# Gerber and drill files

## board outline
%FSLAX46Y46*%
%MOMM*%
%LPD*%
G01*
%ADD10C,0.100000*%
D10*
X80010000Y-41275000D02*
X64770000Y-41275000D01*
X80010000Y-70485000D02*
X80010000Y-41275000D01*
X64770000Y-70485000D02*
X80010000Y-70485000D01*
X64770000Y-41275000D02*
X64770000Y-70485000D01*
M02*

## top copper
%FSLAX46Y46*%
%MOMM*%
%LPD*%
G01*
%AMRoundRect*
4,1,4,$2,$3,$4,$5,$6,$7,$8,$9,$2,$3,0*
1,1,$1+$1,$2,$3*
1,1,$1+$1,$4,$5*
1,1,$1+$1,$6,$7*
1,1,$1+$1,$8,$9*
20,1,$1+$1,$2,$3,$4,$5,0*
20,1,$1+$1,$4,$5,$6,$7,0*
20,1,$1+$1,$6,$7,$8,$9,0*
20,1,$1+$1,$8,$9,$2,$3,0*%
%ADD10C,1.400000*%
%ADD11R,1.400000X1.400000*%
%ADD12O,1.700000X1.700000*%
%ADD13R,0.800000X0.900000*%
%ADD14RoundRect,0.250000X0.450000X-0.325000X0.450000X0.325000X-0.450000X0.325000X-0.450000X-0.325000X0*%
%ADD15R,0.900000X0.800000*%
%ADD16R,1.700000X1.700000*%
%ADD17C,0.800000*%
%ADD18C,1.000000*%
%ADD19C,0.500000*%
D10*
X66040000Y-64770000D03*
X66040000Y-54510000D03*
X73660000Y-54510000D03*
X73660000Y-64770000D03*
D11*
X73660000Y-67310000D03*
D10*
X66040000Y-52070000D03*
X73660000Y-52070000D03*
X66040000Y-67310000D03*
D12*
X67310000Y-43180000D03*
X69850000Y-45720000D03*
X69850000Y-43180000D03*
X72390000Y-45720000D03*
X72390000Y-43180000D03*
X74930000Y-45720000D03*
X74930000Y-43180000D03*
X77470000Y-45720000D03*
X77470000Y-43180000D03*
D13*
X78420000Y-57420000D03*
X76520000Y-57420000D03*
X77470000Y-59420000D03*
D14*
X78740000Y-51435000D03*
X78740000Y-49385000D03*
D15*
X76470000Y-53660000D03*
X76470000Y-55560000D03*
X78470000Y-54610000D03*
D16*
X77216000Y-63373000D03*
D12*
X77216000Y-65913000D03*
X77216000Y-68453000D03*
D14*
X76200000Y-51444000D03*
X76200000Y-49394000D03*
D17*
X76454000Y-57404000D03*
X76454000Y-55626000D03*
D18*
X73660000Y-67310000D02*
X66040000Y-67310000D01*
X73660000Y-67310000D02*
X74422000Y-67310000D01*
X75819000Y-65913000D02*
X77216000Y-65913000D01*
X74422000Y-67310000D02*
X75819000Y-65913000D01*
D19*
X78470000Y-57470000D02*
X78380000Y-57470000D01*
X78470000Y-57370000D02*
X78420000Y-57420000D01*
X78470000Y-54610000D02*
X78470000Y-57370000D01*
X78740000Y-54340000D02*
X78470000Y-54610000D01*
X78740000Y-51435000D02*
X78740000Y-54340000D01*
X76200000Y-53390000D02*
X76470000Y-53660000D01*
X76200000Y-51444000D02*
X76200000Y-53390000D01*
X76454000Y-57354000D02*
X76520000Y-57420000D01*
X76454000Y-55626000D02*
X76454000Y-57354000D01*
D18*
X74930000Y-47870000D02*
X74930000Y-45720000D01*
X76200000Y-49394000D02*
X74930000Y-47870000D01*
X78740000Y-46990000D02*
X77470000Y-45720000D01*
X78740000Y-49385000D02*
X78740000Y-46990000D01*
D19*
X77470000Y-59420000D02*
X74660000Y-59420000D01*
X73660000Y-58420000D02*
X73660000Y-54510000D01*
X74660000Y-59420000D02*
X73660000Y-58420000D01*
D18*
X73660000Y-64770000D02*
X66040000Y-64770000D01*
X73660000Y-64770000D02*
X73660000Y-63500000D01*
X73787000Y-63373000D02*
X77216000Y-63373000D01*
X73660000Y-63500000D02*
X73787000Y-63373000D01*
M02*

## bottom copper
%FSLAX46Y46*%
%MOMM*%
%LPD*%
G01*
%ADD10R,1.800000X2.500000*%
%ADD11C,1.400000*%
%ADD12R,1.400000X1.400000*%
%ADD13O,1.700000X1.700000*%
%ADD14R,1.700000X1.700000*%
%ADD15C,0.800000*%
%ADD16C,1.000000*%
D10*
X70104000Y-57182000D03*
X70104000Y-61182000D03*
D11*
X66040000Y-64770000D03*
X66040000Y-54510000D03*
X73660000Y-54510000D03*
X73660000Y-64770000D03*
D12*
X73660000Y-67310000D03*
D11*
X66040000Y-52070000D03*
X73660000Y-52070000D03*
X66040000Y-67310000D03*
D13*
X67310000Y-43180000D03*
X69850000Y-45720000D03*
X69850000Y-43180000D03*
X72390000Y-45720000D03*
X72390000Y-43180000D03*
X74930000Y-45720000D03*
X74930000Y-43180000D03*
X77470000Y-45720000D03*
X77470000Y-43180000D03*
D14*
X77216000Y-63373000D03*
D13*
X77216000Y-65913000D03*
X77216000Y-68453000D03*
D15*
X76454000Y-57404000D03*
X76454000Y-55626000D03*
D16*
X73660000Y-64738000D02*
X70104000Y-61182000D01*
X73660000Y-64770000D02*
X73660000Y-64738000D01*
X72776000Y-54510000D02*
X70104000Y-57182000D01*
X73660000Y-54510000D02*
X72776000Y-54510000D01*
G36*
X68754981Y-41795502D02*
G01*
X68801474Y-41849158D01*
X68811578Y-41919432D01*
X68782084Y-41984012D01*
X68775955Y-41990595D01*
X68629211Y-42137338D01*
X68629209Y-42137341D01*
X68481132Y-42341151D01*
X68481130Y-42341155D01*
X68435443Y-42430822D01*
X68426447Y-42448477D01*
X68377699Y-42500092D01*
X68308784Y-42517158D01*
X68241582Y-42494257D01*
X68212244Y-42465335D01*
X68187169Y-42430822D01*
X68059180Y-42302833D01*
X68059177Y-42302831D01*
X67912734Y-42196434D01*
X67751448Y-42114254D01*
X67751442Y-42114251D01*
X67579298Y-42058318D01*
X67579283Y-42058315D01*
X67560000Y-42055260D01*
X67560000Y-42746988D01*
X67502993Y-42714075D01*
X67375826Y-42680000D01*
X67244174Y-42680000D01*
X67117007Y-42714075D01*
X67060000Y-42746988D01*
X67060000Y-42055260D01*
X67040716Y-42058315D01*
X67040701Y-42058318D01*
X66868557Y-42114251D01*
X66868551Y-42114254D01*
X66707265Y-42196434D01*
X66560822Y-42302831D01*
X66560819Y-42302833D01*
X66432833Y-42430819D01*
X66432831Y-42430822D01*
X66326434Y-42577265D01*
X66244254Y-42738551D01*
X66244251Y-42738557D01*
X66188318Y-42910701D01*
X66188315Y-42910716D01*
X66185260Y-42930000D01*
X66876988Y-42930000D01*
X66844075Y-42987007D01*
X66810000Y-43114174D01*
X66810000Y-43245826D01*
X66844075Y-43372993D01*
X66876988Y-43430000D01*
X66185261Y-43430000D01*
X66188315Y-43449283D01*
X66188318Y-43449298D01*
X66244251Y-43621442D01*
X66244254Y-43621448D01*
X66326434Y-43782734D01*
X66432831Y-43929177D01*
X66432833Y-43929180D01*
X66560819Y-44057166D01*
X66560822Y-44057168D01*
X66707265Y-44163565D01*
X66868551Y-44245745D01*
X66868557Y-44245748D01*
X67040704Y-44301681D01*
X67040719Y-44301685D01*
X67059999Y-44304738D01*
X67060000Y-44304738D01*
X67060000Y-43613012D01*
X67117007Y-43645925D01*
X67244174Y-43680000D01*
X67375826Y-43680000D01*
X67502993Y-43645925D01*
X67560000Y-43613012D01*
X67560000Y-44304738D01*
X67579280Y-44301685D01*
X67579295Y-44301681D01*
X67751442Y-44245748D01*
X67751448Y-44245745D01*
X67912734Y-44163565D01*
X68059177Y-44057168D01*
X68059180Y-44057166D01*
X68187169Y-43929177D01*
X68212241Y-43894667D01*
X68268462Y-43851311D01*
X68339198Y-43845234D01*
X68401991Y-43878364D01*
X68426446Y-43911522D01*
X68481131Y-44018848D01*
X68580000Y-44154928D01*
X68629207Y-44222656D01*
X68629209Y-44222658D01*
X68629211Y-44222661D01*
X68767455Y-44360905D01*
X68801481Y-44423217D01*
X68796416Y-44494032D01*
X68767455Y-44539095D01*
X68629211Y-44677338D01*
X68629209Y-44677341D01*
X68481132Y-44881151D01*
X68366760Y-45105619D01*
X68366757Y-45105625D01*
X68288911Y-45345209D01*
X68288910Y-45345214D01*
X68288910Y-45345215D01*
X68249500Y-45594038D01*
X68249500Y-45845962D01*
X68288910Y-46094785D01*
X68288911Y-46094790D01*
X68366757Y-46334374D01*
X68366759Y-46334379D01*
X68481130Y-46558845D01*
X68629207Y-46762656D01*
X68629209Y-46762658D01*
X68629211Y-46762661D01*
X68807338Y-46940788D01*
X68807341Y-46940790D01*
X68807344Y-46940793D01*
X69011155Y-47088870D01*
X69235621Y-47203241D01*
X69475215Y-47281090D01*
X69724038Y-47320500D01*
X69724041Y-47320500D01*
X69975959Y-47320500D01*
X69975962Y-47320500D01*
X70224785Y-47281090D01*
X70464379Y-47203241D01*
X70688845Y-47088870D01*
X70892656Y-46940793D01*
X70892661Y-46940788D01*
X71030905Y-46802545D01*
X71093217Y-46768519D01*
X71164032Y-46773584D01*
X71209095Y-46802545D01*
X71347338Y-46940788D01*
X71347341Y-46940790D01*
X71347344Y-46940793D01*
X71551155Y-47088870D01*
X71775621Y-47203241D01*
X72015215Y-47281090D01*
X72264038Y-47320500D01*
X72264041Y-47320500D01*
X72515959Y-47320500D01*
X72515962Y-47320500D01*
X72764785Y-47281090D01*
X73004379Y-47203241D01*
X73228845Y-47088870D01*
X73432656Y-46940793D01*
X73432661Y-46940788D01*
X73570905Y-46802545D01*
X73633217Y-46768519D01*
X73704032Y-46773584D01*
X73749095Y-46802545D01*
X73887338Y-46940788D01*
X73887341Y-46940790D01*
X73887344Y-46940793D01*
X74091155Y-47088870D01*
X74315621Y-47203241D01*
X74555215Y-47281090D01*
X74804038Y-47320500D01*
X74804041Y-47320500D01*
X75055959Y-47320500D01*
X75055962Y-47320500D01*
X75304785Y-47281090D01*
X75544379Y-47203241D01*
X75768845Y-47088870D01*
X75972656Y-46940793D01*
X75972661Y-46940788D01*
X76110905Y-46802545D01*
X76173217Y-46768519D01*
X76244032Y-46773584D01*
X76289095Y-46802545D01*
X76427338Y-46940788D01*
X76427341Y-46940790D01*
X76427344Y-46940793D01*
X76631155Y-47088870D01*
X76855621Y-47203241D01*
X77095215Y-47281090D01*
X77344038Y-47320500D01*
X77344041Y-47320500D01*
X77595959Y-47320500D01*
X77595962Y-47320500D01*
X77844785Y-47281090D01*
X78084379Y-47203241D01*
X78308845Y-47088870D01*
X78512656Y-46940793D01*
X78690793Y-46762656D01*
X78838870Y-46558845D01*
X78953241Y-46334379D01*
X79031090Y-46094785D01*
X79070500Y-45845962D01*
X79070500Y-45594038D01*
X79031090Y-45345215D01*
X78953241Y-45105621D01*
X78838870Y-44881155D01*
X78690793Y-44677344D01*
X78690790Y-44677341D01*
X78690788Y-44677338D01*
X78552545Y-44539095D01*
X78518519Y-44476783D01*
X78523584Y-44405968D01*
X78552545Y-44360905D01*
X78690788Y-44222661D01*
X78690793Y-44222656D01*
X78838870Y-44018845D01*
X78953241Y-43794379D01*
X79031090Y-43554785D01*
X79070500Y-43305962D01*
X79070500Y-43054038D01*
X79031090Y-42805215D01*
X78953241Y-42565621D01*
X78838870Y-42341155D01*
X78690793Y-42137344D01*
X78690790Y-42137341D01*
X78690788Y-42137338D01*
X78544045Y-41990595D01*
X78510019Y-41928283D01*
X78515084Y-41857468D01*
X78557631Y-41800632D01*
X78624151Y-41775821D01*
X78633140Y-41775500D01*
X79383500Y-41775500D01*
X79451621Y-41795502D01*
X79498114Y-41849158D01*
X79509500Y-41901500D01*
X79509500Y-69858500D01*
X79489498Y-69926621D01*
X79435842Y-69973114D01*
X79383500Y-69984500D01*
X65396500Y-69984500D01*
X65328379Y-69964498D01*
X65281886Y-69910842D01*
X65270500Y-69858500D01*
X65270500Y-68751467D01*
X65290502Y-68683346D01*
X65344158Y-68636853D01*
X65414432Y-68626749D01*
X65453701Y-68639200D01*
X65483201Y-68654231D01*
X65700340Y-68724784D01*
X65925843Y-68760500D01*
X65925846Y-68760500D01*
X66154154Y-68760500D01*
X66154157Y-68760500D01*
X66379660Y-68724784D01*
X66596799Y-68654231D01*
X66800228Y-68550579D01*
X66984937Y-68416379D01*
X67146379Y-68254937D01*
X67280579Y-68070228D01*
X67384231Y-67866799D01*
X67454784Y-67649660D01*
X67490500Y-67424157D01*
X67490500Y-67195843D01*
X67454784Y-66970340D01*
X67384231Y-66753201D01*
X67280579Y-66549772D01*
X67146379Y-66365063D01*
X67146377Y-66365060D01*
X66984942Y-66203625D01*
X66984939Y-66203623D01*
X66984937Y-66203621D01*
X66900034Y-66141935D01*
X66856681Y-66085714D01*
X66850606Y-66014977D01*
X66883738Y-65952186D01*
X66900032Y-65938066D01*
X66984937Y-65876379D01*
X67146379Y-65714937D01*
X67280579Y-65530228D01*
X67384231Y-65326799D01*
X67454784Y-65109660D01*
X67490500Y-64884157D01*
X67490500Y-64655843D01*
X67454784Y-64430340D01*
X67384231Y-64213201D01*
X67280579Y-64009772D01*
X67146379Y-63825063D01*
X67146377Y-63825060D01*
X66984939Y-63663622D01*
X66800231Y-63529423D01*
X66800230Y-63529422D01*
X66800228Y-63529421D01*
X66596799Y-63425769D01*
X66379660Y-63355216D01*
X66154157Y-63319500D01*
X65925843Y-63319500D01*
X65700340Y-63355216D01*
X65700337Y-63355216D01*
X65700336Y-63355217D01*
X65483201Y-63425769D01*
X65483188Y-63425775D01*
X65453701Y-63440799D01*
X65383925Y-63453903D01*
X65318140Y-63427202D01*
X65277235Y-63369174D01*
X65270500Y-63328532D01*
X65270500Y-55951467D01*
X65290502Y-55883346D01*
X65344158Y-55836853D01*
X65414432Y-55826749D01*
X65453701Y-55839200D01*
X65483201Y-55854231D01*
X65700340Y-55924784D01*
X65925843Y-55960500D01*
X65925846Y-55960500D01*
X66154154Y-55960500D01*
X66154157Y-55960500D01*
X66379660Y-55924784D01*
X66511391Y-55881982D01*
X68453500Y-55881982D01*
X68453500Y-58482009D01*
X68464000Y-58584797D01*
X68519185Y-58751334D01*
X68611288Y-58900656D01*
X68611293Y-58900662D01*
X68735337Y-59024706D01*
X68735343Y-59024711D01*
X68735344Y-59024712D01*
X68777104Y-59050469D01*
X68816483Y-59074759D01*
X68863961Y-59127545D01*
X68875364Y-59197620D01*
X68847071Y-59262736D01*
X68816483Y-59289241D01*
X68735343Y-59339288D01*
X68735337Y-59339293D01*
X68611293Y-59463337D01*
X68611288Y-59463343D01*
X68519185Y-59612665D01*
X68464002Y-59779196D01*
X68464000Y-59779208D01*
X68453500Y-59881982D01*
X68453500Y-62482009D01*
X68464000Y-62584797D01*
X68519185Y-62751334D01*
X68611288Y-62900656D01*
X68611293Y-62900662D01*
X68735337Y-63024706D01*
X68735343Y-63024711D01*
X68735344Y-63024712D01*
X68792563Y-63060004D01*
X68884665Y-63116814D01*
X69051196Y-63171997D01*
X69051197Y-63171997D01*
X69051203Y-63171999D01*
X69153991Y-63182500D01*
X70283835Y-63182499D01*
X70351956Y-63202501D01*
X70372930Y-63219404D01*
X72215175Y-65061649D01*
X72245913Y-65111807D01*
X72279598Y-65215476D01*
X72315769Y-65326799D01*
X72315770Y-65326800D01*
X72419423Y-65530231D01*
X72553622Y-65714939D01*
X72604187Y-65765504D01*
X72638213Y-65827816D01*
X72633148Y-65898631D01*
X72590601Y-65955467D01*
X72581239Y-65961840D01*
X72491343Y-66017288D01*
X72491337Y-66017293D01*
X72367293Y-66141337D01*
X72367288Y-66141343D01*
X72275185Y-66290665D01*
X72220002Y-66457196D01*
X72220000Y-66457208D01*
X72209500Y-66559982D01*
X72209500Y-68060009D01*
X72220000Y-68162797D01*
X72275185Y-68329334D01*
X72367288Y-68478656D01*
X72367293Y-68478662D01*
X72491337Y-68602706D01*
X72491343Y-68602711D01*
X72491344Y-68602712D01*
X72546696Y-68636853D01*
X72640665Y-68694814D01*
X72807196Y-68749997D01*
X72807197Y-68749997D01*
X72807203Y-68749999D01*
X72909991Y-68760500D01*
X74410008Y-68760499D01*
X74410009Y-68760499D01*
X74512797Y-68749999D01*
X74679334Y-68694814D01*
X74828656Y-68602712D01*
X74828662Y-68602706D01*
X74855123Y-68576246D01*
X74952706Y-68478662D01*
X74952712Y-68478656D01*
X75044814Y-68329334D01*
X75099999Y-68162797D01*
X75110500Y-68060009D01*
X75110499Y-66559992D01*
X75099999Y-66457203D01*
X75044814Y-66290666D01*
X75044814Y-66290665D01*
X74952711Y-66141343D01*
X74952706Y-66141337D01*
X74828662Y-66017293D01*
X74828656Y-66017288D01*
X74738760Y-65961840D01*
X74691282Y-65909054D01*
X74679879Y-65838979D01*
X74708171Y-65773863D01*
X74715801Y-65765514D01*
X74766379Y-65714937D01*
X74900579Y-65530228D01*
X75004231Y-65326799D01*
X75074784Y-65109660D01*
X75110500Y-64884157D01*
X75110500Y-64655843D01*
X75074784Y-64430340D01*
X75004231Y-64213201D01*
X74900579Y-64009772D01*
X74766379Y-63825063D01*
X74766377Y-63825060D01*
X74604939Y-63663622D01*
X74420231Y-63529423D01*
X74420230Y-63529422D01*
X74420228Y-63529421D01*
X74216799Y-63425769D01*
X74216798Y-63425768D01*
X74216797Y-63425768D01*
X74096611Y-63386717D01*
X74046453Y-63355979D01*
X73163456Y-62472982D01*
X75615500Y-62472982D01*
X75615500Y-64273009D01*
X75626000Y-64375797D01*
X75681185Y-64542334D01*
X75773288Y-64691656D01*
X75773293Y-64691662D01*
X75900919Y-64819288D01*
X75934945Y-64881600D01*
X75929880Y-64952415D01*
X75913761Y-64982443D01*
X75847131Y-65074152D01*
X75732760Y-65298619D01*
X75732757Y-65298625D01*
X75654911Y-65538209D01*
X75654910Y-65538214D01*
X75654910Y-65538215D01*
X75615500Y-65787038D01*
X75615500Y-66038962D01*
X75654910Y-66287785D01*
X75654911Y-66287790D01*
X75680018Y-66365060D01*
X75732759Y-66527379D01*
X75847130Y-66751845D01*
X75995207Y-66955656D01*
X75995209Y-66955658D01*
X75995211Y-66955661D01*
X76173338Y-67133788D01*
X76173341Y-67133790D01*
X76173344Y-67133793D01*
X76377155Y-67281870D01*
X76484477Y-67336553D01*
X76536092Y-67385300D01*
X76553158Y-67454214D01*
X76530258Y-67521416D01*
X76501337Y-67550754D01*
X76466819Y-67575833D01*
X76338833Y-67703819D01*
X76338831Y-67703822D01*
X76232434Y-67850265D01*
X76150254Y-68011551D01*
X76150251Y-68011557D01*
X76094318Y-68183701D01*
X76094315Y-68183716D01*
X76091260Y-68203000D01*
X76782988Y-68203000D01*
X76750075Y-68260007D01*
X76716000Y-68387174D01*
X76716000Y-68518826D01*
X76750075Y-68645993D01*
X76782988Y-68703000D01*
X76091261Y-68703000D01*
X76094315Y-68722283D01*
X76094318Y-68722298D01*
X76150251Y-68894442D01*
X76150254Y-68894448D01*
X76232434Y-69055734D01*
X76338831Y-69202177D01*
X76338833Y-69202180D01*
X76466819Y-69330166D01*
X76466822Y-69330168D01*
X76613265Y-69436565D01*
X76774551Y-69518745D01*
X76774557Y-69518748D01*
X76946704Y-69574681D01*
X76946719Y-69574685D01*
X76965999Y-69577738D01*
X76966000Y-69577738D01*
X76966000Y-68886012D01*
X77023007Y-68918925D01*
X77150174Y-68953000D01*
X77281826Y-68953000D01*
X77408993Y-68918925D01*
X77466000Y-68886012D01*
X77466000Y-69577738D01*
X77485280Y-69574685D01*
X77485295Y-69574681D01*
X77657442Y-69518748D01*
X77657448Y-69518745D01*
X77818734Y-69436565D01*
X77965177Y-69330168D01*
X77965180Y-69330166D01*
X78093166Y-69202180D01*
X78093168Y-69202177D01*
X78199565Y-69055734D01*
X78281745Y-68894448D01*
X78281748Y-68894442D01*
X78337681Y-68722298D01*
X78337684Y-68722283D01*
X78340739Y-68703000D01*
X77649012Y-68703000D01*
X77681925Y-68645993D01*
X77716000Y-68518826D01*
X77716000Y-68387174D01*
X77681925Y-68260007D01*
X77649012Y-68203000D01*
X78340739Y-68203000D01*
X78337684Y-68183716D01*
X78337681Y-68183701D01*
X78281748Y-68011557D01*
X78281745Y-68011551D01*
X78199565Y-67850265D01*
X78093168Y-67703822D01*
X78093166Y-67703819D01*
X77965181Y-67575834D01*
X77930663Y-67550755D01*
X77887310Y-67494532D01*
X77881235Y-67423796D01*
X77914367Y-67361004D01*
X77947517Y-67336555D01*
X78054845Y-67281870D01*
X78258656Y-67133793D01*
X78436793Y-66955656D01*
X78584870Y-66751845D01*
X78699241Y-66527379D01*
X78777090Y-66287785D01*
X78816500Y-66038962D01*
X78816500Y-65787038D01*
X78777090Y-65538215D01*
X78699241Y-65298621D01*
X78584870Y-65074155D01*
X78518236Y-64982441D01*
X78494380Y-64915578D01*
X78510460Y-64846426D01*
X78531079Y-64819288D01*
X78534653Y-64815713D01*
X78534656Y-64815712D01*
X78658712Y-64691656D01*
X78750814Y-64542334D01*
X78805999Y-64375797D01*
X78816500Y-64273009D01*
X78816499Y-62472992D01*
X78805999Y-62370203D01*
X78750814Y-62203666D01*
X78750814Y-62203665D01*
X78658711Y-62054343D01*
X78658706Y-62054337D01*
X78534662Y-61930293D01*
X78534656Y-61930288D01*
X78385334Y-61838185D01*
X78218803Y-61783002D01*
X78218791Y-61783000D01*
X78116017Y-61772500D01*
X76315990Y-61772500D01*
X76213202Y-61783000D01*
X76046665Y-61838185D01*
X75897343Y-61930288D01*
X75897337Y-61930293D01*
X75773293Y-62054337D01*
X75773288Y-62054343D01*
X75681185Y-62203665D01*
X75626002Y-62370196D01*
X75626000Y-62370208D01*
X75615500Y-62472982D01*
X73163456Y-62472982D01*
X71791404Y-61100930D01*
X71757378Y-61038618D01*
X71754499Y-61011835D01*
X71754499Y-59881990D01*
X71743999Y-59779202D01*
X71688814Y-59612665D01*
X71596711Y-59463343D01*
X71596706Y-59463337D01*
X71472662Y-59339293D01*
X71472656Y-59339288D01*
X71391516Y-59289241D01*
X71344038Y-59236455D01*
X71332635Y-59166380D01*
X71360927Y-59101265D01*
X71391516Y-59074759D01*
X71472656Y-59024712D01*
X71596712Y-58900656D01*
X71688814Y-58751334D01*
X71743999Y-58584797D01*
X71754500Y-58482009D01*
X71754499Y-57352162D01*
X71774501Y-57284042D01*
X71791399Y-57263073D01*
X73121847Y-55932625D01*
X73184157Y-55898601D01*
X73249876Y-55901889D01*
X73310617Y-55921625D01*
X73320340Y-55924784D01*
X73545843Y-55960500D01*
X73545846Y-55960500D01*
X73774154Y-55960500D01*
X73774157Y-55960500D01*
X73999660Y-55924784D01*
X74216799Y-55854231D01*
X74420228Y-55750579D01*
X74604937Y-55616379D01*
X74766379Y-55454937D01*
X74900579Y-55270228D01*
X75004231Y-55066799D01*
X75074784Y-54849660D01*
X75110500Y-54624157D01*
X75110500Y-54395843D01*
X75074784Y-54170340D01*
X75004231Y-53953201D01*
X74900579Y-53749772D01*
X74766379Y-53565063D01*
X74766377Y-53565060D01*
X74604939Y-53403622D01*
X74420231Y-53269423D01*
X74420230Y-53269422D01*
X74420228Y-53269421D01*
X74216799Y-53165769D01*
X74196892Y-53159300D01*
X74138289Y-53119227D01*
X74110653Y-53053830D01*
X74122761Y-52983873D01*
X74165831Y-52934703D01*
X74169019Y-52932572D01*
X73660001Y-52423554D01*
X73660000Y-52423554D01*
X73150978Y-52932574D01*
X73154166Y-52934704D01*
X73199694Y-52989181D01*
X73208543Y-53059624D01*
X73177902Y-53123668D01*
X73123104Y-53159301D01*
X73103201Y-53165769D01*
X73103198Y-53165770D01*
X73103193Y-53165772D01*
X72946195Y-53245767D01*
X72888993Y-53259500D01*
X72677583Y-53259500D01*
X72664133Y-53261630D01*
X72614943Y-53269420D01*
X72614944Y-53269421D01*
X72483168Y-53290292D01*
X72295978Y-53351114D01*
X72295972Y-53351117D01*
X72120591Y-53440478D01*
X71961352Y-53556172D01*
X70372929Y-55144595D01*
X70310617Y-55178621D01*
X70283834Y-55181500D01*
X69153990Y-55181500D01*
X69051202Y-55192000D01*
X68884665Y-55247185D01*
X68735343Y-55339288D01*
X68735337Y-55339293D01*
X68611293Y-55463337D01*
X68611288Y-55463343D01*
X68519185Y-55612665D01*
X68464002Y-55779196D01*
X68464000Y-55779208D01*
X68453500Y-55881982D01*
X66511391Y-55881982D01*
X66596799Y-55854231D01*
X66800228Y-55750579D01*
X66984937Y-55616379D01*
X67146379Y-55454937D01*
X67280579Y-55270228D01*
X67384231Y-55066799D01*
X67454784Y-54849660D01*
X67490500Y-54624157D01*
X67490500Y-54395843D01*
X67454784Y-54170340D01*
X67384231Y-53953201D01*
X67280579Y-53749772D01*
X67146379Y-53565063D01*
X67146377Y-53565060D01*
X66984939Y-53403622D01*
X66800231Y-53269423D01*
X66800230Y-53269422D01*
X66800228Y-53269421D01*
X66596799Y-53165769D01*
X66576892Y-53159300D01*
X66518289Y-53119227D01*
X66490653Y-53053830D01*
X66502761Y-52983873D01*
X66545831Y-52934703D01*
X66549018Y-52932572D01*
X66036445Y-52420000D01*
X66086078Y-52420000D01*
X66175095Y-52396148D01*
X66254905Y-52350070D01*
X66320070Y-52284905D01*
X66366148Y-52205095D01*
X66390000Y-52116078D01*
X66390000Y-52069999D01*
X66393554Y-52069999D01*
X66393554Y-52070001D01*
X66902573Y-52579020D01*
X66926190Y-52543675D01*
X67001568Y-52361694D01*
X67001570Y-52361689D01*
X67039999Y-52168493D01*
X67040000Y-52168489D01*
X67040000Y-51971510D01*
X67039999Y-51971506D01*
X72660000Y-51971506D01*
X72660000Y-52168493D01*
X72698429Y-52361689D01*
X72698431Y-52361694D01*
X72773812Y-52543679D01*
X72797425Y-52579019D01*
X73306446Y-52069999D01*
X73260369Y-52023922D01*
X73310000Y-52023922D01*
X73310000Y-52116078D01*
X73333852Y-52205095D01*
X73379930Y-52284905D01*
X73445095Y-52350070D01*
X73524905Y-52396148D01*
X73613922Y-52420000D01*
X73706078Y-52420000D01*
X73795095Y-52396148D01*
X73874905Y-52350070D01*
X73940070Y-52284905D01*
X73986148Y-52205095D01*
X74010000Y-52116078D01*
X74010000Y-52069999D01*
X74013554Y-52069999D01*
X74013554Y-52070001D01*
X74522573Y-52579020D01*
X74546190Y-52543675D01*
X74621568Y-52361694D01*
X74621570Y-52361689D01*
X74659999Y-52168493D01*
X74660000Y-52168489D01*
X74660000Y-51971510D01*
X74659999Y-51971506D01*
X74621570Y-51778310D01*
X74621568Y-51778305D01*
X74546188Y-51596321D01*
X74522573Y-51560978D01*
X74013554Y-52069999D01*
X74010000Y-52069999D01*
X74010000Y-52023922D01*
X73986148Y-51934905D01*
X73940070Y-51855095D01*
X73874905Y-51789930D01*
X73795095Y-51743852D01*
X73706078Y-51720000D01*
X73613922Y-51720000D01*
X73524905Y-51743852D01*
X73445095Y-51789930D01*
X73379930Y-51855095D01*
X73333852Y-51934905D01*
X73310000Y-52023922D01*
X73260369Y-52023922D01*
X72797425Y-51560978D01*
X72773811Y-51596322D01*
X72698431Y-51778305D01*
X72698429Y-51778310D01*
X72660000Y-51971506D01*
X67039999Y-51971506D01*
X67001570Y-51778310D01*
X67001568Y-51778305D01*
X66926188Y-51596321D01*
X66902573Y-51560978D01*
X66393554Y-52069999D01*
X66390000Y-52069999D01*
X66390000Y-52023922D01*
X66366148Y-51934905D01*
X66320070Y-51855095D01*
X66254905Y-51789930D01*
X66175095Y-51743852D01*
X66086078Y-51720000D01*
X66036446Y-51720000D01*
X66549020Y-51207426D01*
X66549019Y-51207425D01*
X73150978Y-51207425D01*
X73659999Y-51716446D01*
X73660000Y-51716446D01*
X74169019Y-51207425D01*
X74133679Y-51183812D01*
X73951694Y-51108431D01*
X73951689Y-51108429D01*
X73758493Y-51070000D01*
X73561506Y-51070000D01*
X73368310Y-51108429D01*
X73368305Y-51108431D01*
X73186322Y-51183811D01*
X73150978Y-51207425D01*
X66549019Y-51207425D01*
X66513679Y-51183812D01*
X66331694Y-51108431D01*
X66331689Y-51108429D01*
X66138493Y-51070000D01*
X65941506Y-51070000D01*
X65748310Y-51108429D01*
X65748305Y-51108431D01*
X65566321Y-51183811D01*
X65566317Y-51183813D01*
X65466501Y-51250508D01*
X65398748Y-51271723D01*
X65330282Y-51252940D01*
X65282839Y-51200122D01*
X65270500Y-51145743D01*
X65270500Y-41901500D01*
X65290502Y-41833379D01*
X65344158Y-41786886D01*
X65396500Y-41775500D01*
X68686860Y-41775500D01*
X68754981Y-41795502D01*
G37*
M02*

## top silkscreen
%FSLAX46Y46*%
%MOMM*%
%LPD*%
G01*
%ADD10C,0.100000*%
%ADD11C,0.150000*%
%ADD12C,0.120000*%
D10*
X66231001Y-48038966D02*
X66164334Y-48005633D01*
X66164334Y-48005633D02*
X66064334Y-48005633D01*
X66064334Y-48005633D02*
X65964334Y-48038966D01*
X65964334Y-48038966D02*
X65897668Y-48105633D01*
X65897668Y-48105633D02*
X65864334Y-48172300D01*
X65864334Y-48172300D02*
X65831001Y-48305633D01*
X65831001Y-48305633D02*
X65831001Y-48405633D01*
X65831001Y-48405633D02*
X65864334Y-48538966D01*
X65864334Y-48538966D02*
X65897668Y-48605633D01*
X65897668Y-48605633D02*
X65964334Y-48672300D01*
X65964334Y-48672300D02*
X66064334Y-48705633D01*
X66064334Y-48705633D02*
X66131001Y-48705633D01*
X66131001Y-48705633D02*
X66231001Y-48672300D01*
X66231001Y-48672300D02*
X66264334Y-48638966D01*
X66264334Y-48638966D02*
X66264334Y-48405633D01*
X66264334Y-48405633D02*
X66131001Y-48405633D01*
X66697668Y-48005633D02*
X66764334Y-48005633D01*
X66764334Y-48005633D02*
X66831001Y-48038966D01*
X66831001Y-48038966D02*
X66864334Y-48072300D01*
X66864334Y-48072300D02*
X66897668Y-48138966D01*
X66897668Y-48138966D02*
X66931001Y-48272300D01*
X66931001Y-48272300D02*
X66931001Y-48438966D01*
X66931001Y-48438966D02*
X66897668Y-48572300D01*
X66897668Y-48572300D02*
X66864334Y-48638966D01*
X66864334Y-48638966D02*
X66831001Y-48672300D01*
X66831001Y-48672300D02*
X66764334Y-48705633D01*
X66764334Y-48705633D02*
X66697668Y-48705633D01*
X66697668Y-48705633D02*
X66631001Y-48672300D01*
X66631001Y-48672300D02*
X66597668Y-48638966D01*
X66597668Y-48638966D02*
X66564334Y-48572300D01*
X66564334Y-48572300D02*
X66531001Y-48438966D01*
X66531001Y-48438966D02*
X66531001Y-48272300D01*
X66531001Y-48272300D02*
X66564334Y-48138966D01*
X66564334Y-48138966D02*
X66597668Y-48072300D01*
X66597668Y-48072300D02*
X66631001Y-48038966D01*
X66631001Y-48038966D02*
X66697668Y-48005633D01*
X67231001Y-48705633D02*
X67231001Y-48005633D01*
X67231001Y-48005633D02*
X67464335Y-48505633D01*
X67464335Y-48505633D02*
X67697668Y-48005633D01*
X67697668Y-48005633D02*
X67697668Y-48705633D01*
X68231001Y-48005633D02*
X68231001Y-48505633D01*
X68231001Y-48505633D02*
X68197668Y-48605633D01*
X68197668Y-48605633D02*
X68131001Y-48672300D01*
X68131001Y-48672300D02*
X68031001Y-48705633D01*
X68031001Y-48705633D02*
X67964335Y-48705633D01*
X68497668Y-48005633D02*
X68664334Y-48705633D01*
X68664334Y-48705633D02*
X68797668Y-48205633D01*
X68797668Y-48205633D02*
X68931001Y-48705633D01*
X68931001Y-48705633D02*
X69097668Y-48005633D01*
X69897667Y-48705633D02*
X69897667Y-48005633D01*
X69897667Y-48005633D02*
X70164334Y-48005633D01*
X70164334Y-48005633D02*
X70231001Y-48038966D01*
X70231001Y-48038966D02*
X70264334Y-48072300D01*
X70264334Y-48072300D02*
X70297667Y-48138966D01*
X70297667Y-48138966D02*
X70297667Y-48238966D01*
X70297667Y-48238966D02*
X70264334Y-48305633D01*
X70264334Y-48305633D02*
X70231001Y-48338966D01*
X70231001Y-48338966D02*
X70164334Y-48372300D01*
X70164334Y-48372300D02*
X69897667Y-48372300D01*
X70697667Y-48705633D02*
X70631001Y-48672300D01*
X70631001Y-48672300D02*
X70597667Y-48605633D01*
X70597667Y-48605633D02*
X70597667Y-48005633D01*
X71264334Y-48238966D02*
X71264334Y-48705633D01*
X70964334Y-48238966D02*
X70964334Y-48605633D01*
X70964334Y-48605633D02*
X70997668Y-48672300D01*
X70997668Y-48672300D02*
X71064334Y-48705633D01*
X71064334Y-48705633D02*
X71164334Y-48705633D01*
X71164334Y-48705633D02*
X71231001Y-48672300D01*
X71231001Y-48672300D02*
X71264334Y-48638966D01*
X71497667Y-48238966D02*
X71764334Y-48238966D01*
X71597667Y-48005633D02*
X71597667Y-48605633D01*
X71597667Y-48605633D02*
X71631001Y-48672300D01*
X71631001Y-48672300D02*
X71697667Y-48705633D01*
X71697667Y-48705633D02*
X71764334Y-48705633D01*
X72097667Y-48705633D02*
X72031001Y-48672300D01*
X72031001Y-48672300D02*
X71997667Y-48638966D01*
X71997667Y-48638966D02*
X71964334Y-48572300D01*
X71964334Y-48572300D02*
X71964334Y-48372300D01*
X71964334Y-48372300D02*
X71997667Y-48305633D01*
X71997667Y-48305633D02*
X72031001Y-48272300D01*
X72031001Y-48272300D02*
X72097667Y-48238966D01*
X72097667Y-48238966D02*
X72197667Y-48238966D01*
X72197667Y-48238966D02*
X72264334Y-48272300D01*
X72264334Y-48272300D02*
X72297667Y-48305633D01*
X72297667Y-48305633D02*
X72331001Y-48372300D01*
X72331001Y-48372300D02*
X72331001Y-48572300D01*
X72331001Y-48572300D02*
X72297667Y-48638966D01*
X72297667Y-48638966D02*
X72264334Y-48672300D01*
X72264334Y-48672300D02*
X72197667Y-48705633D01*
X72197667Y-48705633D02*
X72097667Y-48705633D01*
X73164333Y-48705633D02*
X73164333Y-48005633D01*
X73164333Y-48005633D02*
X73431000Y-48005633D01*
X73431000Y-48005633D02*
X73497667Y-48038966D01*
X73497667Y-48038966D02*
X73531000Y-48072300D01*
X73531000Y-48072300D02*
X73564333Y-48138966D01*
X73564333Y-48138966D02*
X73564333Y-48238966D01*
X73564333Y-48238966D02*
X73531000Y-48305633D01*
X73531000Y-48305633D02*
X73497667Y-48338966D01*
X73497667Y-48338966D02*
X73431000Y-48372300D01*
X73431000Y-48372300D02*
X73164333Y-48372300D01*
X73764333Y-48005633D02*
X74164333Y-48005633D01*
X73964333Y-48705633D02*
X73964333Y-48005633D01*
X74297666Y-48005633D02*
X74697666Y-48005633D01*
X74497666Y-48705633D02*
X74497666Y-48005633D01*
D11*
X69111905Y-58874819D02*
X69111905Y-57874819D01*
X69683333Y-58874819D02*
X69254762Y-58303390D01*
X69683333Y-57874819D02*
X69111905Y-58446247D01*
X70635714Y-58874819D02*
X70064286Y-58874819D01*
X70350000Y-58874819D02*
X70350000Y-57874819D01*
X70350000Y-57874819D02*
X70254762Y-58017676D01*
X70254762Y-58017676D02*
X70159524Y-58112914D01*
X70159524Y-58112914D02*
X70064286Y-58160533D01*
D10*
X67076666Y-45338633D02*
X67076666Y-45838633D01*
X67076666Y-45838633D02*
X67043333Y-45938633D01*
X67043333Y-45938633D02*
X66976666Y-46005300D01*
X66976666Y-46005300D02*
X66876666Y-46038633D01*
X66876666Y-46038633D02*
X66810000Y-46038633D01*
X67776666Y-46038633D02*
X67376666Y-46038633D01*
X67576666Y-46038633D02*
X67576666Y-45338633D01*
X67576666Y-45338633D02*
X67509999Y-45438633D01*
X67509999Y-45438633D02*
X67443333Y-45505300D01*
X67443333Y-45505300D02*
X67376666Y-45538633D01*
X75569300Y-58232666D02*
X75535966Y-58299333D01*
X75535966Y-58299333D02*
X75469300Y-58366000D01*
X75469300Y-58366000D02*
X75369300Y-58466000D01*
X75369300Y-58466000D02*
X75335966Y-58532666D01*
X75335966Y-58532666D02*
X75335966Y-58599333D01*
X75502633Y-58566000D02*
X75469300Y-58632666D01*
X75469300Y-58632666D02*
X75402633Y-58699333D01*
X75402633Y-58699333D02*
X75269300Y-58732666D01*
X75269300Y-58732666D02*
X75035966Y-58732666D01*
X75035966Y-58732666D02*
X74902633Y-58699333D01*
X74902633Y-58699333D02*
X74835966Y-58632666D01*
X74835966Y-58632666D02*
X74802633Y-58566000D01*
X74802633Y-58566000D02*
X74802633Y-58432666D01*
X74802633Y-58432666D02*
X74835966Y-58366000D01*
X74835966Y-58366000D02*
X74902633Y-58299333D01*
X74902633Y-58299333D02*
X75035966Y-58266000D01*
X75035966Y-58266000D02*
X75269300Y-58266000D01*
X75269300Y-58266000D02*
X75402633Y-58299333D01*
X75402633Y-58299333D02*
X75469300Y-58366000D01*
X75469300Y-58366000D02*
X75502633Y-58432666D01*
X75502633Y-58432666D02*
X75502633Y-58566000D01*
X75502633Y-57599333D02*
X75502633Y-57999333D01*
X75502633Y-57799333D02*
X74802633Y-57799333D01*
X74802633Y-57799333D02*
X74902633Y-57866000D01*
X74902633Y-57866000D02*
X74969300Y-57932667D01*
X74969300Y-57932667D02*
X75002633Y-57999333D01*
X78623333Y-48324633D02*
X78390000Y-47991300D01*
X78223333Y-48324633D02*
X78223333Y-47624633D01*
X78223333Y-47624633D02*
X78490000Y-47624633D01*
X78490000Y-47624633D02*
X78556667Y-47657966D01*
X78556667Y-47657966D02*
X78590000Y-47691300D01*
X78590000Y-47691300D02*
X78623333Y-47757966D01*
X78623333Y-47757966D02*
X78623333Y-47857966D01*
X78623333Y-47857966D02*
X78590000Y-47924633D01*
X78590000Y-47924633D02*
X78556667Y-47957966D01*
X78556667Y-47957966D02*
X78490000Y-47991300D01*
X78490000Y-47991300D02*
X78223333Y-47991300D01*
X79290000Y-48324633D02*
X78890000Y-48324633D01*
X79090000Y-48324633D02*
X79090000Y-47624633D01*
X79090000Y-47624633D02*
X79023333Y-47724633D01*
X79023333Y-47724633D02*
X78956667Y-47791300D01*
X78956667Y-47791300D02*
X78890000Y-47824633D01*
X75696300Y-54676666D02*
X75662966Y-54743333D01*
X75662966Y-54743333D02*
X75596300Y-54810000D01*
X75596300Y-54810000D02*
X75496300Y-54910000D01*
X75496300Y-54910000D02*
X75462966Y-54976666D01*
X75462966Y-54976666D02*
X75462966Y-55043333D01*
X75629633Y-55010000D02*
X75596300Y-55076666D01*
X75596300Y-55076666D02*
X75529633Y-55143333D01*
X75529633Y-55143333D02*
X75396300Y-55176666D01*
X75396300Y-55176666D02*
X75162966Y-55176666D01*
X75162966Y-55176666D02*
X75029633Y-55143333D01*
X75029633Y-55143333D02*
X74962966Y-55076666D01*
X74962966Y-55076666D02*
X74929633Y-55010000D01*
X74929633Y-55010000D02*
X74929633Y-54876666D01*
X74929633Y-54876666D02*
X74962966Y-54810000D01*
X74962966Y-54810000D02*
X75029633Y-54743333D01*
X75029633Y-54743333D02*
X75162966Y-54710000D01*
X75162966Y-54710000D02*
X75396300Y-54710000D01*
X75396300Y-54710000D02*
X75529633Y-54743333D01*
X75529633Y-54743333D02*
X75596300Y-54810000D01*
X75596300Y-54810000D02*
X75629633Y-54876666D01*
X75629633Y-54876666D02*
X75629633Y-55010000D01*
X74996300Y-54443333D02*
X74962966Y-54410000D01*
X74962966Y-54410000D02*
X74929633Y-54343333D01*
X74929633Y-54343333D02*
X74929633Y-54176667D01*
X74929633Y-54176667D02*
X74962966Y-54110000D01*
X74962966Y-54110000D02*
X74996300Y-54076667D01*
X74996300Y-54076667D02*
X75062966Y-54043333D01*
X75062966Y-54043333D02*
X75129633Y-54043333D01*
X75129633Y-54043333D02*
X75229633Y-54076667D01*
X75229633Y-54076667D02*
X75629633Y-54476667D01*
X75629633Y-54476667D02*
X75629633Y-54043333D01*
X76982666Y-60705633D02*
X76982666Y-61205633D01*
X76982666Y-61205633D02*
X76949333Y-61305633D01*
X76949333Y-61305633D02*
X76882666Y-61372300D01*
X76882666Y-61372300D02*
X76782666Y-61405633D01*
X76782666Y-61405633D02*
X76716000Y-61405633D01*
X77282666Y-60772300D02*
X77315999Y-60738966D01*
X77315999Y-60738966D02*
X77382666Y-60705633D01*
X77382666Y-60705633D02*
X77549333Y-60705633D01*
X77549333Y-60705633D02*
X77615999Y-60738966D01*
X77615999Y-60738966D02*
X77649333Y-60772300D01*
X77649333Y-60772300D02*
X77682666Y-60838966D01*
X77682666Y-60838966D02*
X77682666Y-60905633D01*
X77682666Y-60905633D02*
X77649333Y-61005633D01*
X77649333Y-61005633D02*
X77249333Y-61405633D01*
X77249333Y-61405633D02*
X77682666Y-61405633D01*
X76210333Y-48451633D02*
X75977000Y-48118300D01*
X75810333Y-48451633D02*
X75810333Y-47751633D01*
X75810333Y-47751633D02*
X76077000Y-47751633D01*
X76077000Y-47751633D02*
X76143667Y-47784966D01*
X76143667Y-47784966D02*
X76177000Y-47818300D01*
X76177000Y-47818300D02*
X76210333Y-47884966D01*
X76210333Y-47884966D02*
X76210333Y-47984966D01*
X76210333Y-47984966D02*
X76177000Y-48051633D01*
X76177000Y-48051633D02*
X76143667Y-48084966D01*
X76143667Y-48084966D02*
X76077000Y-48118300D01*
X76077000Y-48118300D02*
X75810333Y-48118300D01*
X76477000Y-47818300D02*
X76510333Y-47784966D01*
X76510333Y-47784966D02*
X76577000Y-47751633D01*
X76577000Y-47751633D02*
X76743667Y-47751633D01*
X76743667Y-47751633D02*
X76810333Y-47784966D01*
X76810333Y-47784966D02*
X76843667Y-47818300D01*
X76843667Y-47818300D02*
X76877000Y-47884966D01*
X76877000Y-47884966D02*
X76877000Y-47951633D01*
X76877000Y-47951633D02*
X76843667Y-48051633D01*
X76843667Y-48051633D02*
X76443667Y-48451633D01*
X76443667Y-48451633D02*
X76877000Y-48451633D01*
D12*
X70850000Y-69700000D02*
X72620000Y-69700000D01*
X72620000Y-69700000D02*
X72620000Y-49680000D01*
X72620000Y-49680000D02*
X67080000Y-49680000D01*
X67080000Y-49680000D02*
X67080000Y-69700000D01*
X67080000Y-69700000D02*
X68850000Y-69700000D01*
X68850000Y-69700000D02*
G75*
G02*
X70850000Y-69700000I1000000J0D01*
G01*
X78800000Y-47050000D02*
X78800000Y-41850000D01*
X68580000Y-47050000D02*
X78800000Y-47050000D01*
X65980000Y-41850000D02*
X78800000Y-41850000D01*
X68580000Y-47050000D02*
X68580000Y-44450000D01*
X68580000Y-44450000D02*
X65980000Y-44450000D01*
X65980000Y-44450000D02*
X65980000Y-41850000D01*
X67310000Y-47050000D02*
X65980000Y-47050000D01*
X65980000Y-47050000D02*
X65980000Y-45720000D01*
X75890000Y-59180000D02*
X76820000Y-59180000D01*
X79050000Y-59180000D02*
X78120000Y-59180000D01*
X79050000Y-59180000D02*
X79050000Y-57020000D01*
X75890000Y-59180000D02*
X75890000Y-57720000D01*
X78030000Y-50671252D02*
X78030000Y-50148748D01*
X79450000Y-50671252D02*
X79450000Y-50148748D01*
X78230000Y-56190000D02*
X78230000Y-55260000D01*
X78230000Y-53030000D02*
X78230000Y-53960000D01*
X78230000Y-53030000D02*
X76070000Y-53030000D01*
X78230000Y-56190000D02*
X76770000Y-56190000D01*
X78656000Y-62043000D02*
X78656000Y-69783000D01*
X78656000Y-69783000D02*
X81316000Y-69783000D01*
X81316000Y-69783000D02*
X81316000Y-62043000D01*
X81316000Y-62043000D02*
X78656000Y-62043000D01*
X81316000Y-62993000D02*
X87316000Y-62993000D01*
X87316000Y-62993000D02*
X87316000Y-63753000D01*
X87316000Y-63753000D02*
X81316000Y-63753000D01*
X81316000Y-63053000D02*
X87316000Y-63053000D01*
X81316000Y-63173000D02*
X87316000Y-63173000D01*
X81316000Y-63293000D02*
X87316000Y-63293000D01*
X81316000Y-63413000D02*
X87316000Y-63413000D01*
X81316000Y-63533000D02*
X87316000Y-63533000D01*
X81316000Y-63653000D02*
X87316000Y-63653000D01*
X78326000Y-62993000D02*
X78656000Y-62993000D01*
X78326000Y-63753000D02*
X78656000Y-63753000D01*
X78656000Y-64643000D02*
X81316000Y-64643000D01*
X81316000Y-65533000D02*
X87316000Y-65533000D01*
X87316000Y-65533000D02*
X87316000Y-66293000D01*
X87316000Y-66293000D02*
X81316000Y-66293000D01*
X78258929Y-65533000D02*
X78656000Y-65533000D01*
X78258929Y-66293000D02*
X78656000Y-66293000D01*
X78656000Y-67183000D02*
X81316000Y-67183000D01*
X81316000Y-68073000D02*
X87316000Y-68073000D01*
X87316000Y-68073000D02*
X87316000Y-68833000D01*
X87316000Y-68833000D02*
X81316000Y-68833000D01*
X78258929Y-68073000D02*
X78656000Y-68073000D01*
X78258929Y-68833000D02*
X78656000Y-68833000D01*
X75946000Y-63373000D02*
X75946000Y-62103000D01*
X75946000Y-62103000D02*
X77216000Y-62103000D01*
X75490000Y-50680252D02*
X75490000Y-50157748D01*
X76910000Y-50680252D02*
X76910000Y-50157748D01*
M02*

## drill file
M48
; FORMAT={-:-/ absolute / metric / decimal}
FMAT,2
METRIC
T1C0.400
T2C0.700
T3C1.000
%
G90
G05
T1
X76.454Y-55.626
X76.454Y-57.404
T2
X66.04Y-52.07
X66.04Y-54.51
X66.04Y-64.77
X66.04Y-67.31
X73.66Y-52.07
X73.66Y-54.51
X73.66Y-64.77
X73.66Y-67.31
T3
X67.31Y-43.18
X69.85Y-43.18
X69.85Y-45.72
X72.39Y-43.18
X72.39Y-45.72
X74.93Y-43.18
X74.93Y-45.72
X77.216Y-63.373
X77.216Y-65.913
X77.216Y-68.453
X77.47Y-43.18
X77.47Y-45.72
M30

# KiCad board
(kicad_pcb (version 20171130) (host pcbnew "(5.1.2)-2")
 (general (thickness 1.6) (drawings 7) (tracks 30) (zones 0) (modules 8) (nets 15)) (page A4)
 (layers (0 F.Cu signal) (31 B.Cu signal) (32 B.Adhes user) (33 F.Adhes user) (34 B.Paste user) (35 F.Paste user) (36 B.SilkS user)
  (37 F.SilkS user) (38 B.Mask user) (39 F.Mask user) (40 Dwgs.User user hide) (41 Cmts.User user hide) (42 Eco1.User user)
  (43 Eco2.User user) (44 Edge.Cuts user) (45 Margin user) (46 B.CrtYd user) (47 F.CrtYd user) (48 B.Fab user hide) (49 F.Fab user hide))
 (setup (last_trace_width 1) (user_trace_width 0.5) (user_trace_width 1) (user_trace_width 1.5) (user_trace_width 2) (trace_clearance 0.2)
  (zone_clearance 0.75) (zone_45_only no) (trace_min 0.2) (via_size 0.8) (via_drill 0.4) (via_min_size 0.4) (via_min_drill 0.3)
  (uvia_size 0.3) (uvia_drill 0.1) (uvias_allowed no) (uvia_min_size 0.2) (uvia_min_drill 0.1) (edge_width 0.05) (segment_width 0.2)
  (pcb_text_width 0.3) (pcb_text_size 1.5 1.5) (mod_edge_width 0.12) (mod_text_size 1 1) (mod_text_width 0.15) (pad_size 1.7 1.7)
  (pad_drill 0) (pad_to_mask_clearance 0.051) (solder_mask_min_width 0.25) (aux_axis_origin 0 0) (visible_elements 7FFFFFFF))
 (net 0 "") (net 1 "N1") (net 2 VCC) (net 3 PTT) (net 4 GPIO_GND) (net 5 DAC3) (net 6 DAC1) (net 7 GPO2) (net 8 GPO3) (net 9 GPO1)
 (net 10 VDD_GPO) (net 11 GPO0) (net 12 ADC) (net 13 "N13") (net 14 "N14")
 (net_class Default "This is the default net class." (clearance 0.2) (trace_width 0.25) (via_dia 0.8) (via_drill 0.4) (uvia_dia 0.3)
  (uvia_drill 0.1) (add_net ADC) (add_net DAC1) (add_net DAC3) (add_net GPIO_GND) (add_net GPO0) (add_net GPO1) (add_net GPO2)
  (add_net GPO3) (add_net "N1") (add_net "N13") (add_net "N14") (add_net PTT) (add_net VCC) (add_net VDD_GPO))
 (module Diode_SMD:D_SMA (layer B.Cu) (at 70.104 59.182 90)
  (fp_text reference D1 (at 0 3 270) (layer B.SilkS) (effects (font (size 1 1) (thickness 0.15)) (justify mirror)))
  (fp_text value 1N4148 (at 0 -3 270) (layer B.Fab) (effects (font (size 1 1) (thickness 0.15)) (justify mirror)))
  (pad 2 smd rect (at 2 0 90) (size 2.5 1.8) (layers B.Cu B.Paste B.Mask) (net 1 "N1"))
  (pad 1 smd rect (at -2 0 90) (size 2.5 1.8) (layers B.Cu B.Paste B.Mask) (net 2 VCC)))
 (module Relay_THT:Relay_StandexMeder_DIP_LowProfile (layer F.Cu) (at 73.66 67.31 180)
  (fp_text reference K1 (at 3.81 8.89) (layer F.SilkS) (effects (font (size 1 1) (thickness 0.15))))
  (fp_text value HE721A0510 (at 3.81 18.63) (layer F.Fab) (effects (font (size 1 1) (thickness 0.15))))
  (fp_line (start 2.81 -2.39) (end 1.04 -2.39) (layer F.SilkS) (width 0.12))
  (fp_line (start 1.04 -2.39) (end 1.04 17.63) (layer F.SilkS) (width 0.12))
  (fp_line (start 1.04 17.63) (end 6.58 17.63) (layer F.SilkS) (width 0.12))
  (fp_line (start 6.58 17.63) (end 6.58 -2.39) (layer F.SilkS) (width 0.12))
  (fp_line (start 6.58 -2.39) (end 4.81 -2.39) (layer F.SilkS) (width 0.12))
  (fp_arc (start 3.81 -2.39) (end 2.81 -2.39) (angle -180) (layer F.SilkS) (width 0.12))
  (pad 13 thru_hole circle (at 7.62 2.54 180) (size 1.4 1.4) (drill 0.7) (layers *.Cu *.Mask) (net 2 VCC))
  (pad 9 thru_hole circle (at 7.62 12.8 180) (size 1.4 1.4) (drill 0.7) (layers *.Cu *.Mask))
  (pad 6 thru_hole circle (at 0 12.8 180) (size 1.4 1.4) (drill 0.7) (layers *.Cu *.Mask) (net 1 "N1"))
  (pad 2 thru_hole circle (at 0 2.54 180) (size 1.4 1.4) (drill 0.7) (layers *.Cu *.Mask) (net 2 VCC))
  (pad 1 thru_hole rect (at 0 0 180) (size 1.4 1.4) (drill 0.7) (layers *.Cu *.Mask) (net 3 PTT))
  (pad 8 thru_hole circle (at 7.62 15.24 180) (size 1.4 1.4) (drill 0.7) (layers *.Cu *.Mask) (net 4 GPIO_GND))
  (pad 7 thru_hole circle (at 0 15.24 180) (size 1.4 1.4) (drill 0.7) (layers *.Cu *.Mask) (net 4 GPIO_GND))
  (pad 14 thru_hole circle (at 7.62 0 180) (size 1.4 1.4) (drill 0.7) (layers *.Cu *.Mask) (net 3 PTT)))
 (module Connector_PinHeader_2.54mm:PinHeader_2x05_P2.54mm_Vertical (layer F.Cu) (at 67.31 45.72 90)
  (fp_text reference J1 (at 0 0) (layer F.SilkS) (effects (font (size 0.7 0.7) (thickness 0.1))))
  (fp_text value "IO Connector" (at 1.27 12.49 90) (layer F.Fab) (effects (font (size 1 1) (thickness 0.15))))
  (fp_line (start -1.33 11.49) (end 3.87 11.49) (layer F.SilkS) (width 0.12))
  (fp_line (start -1.33 1.27) (end -1.33 11.49) (layer F.SilkS) (width 0.12))
  (fp_line (start 3.87 -1.33) (end 3.87 11.49) (layer F.SilkS) (width 0.12))
  (fp_line (start -1.33 1.27) (end 1.27 1.27) (layer F.SilkS) (width 0.12))
  (fp_line (start 1.27 1.27) (end 1.27 -1.33) (layer F.SilkS) (width 0.12))
  (fp_line (start 1.27 -1.33) (end 3.87 -1.33) (layer F.SilkS) (width 0.12))
  (fp_line (start -1.33 0) (end -1.33 -1.33) (layer F.SilkS) (width 0.12))
  (fp_line (start -1.33 -1.33) (end 0 -1.33) (layer F.SilkS) (width 0.12))
  (pad 2 thru_hole oval (at 2.54 0 90) (size 1.7 1.7) (drill 1) (layers *.Cu *.Mask) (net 4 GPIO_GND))
  (pad 3 thru_hole oval (at 0 2.54 90) (size 1.7 1.7) (drill 1) (layers *.Cu *.Mask) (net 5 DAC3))
  (pad 4 thru_hole oval (at 2.54 2.54 90) (size 1.7 1.7) (drill 1) (layers *.Cu *.Mask) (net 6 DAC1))
  (pad 5 thru_hole oval (at 0 5.08 90) (size 1.7 1.7) (drill 1) (layers *.Cu *.Mask) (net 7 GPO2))
  (pad 6 thru_hole oval (at 2.54 5.08 90) (size 1.7 1.7) (drill 1) (layers *.Cu *.Mask) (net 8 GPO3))
  (pad 7 thru_hole oval (at 0 7.62 90) (size 1.7 1.7) (drill 1) (layers *.Cu *.Mask) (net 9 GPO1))
  (pad 8 thru_hole oval (at 2.54 7.62 90) (size 1.7 1.7) (drill 1) (layers *.Cu *.Mask) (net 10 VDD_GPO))
  (pad 9 thru_hole oval (at 0 10.16 90) (size 1.7 1.7) (drill 1) (layers *.Cu *.Mask) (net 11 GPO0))
  (pad 10 thru_hole oval (at 2.54 10.16 90) (size 1.7 1.7) (drill 1) (layers *.Cu *.Mask) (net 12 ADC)))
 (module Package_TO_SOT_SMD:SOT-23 (layer F.Cu) (at 77.47 58.42 270)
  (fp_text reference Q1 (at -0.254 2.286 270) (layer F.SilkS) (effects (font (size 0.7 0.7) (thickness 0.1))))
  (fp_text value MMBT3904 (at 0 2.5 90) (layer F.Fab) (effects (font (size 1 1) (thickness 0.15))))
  (fp_line (start 0.76 1.58) (end 0.76 0.65) (layer F.SilkS) (width 0.12))
  (fp_line (start 0.76 -1.58) (end 0.76 -0.65) (layer F.SilkS) (width 0.12))
  (fp_line (start 0.76 -1.58) (end -1.4 -1.58) (layer F.SilkS) (width 0.12))
  (fp_line (start 0.76 1.58) (end -0.7 1.58) (layer F.SilkS) (width 0.12))
  (pad 1 smd rect (at -1 -0.95 270) (size 0.9 0.8) (layers F.Cu F.Paste F.Mask) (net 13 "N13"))
  (pad 2 smd rect (at -1 0.95 270) (size 0.9 0.8) (layers F.Cu F.Paste F.Mask) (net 4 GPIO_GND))
  (pad 3 smd rect (at 1 0 270) (size 0.9 0.8) (layers F.Cu F.Paste F.Mask) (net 1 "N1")))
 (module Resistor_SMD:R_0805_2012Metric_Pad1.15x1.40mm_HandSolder (layer F.Cu) (at 78.74 50.41 90)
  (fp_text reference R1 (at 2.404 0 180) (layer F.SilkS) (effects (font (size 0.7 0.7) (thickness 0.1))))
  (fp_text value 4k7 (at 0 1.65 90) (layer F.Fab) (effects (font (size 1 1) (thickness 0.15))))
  (fp_line (start -0.261252 -0.71) (end 0.261252 -0.71) (layer F.SilkS) (width 0.12))
  (fp_line (start -0.261252 0.71) (end 0.261252 0.71) (layer F.SilkS) (width 0.12))
  (pad 1 smd roundrect (at -1.025 0 90) (size 1.15 1.4) (layers F.Cu F.Paste F.Mask) (roundrect_rratio 0.217391) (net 13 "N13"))
  (pad 2 smd roundrect (at 1.025 0 90) (size 1.15 1.4) (layers F.Cu F.Paste F.Mask) (roundrect_rratio 0.217391) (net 11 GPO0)))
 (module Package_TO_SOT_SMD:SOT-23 (layer F.Cu) (at 77.47 54.61)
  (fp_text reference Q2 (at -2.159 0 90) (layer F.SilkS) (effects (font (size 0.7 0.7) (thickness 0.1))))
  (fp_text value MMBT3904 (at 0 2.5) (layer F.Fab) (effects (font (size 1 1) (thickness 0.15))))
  (fp_line (start 0.76 1.58) (end 0.76 0.65) (layer F.SilkS) (width 0.12))
  (fp_line (start 0.76 -1.58) (end 0.76 -0.65) (layer F.SilkS) (width 0.12))
  (fp_line (start 0.76 -1.58) (end -1.4 -1.58) (layer F.SilkS) (width 0.12))
  (fp_line (start 0.76 1.58) (end -0.7 1.58) (layer F.SilkS) (width 0.12))
  (pad 1 smd rect (at -1 -0.95) (size 0.9 0.8) (layers F.Cu F.Paste F.Mask) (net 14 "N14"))
  (pad 2 smd rect (at -1 0.95) (size 0.9 0.8) (layers F.Cu F.Paste F.Mask) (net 4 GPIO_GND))
  (pad 3 smd rect (at 1 0) (size 0.9 0.8) (layers F.Cu F.Paste F.Mask) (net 13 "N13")))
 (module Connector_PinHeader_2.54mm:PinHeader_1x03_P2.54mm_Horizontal (layer F.Cu) (at 77.216 63.373)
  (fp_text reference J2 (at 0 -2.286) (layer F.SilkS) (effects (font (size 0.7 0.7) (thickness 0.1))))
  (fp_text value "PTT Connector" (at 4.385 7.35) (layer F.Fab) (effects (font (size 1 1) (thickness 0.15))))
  (fp_line (start 1.44 -1.33) (end 1.44 6.41) (layer F.SilkS) (width 0.12))
  (fp_line (start 1.44 6.41) (end 4.1 6.41) (layer F.SilkS) (width 0.12))
  (fp_line (start 4.1 6.41) (end 4.1 -1.33) (layer F.SilkS) (width 0.12))
  (fp_line (start 4.1 -1.33) (end 1.44 -1.33) (layer F.SilkS) (width 0.12))
  (fp_line (start 4.1 -0.38) (end 10.1 -0.38) (layer F.SilkS) (width 0.12))
  (fp_line (start 10.1 -0.38) (end 10.1 0.38) (layer F.SilkS) (width 0.12))
  (fp_line (start 10.1 0.38) (end 4.1 0.38) (layer F.SilkS) (width 0.12))
  (fp_line (start 4.1 -0.32) (end 10.1 -0.32) (layer F.SilkS) (width 0.12))
  (fp_line (start 4.1 -0.2) (end 10.1 -0.2) (layer F.SilkS) (width 0.12))
  (fp_line (start 4.1 -0.08) (end 10.1 -0.08) (layer F.SilkS) (width 0.12))
  (fp_line (start 4.1 0.04) (end 10.1 0.04) (layer F.SilkS) (width 0.12))
  (fp_line (start 4.1 0.16) (end 10.1 0.16) (layer F.SilkS) (width 0.12))
  (fp_line (start 4.1 0.28) (end 10.1 0.28) (layer F.SilkS) (width 0.12))
  (fp_line (start 1.11 -0.38) (end 1.44 -0.38) (layer F.SilkS) (width 0.12))
  (fp_line (start 1.11 0.38) (end 1.44 0.38) (layer F.SilkS) (width 0.12))
  (fp_line (start 1.44 1.27) (end 4.1 1.27) (layer F.SilkS) (width 0.12))
  (fp_line (start 4.1 2.16) (end 10.1 2.16) (layer F.SilkS) (width 0.12))
  (fp_line (start 10.1 2.16) (end 10.1 2.92) (layer F.SilkS) (width 0.12))
  (fp_line (start 10.1 2.92) (end 4.1 2.92) (layer F.SilkS) (width 0.12))
  (fp_line (start 1.042929 2.16) (end 1.44 2.16) (layer F.SilkS) (width 0.12))
  (fp_line (start 1.042929 2.92) (end 1.44 2.92) (layer F.SilkS) (width 0.12))
  (fp_line (start 1.44 3.81) (end 4.1 3.81) (layer F.SilkS) (width 0.12))
  (fp_line (start 4.1 4.7) (end 10.1 4.7) (layer F.SilkS) (width 0.12))
  (fp_line (start 10.1 4.7) (end 10.1 5.46) (layer F.SilkS) (width 0.12))
  (fp_line (start 10.1 5.46) (end 4.1 5.46) (layer F.SilkS) (width 0.12))
  (fp_line (start 1.042929 4.7) (end 1.44 4.7) (layer F.SilkS) (width 0.12))
  (fp_line (start 1.042929 5.46) (end 1.44 5.46) (layer F.SilkS) (width 0.12))
  (fp_line (start -1.27 0) (end -1.27 -1.27) (layer F.SilkS) (width 0.12))
  (fp_line (start -1.27 -1.27) (end 0 -1.27) (layer F.SilkS) (width 0.12))
  (pad 1 thru_hole rect (at 0 0) (size 1.7 1.7) (drill 1) (layers *.Cu *.Mask) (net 2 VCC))
  (pad 2 thru_hole oval (at 0 2.54) (size 1.7 1.7) (drill 1) (layers *.Cu *.Mask) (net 3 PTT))
  (pad 3 thru_hole oval (at 0 5.08) (size 1.7 1.7) (drill 1) (layers *.Cu *.Mask) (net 4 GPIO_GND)))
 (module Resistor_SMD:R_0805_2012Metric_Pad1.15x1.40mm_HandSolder (layer F.Cu) (at 76.2 50.419 90)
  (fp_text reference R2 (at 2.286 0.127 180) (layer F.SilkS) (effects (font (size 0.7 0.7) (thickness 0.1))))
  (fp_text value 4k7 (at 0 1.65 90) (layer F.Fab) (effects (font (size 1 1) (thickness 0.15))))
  (fp_line (start -0.261252 -0.71) (end 0.261252 -0.71) (layer F.SilkS) (width 0.12))
  (fp_line (start -0.261252 0.71) (end 0.261252 0.71) (layer F.SilkS) (width 0.12))
  (pad 1 smd roundrect (at -1.025 0 90) (size 1.15 1.4) (layers F.Cu F.Paste F.Mask) (roundrect_rratio 0.217391) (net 14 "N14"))
  (pad 2 smd roundrect (at 1.025 0 90) (size 1.15 1.4) (layers F.Cu F.Paste F.Mask) (roundrect_rratio 0.217391) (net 9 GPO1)))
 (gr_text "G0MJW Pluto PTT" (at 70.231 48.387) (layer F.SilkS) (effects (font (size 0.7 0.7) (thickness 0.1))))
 (gr_line (start 80.01 41.275) (end 64.77 41.275) (layer Edge.Cuts) (width 0.1))
 (gr_line (start 80.01 70.485) (end 80.01 41.275) (layer Edge.Cuts) (width 0.1))
 (gr_line (start 64.77 70.485) (end 80.01 70.485) (layer Edge.Cuts) (width 0.1))
 (gr_line (start 64.77 41.275) (end 64.77 70.485) (layer Edge.Cuts) (width 0.1))
 (via (at 76.454 57.404) (size 0.8) (drill 0.4) (layers F.Cu B.Cu) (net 4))
 (via (at 76.454 55.626) (size 0.8) (drill 0.4) (layers F.Cu B.Cu) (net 4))
 (segment (start 73.66 67.31) (end 66.04 67.31) (width 1) (layer F.Cu) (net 3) (status 30))
 (segment (start 73.66 67.31) (end 74.422 67.31) (width 1) (layer F.Cu) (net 3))
 (segment (start 75.819 65.913) (end 77.216 65.913) (width 1) (layer F.Cu) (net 3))
 (segment (start 74.422 67.31) (end 75.819 65.913) (width 1) (layer F.Cu) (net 3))
 (segment (start 78.47 57.47) (end 78.38 57.47) (width 0.5) (layer F.Cu) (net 13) (status 30))
 (segment (start 78.47 57.37) (end 78.42 57.42) (width 0.5) (layer F.Cu) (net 13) (status 30))
 (segment (start 78.47 54.61) (end 78.47 57.37) (width 0.5) (layer F.Cu) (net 13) (status 30))
 (segment (start 78.74 54.34) (end 78.47 54.61) (width 0.5) (layer F.Cu) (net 13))
 (segment (start 78.74 51.435) (end 78.74 54.34) (width 0.5) (layer F.Cu) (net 13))
 (segment (start 76.2 53.39) (end 76.47 53.66) (width 0.5) (layer F.Cu) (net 14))
 (segment (start 76.2 51.444) (end 76.2 53.39) (width 0.5) (layer F.Cu) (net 14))
 (segment (start 76.454 57.354) (end 76.52 57.42) (width 0.5) (layer F.Cu) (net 4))
 (segment (start 76.454 55.626) (end 76.454 57.354) (width 0.5) (layer F.Cu) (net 4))
 (segment (start 74.93 47.87) (end 74.93 45.72) (width 1) (layer F.Cu) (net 9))
 (segment (start 76.2 49.394) (end 74.93 47.87) (width 1) (layer F.Cu) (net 9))
 (segment (start 78.74 46.99) (end 77.47 45.72) (width 1) (layer F.Cu) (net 11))
 (segment (start 78.74 49.385) (end 78.74 46.99) (width 1) (layer F.Cu) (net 11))
 (segment (start 77.47 59.42) (end 74.66 59.42) (width 0.5) (layer F.Cu) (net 1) (status 10))
 (segment (start 73.66 58.42) (end 73.66 54.51) (width 0.5) (layer F.Cu) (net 1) (status 20))
 (segment (start 74.66 59.42) (end 73.66 58.42) (width 0.5) (layer F.Cu) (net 1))
 (segment (start 73.66 64.77) (end 66.04 64.77) (width 1) (layer F.Cu) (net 2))
 (segment (start 73.66 64.77) (end 73.66 63.5) (width 1) (layer F.Cu) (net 2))
 (segment (start 73.787 63.373) (end 77.216 63.373) (width 1) (layer F.Cu) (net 2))
 (segment (start 73.66 63.5) (end 73.787 63.373) (width 1) (layer F.Cu) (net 2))
 (segment (start 73.66 64.738) (end 70.104 61.182) (width 1) (layer B.Cu) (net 2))
 (segment (start 73.66 64.77) (end 73.66 64.738) (width 1) (layer B.Cu) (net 2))
 (segment (start 72.776 54.51) (end 70.104 57.182) (width 1) (layer B.Cu) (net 1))
 (segment (start 73.66 54.51) (end 72.776 54.51) (width 1) (layer B.Cu) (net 1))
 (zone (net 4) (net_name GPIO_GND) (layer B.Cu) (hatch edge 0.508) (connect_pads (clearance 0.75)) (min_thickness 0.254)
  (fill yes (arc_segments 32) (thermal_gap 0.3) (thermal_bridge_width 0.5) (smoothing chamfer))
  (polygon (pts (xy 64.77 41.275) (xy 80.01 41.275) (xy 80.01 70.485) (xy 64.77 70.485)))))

